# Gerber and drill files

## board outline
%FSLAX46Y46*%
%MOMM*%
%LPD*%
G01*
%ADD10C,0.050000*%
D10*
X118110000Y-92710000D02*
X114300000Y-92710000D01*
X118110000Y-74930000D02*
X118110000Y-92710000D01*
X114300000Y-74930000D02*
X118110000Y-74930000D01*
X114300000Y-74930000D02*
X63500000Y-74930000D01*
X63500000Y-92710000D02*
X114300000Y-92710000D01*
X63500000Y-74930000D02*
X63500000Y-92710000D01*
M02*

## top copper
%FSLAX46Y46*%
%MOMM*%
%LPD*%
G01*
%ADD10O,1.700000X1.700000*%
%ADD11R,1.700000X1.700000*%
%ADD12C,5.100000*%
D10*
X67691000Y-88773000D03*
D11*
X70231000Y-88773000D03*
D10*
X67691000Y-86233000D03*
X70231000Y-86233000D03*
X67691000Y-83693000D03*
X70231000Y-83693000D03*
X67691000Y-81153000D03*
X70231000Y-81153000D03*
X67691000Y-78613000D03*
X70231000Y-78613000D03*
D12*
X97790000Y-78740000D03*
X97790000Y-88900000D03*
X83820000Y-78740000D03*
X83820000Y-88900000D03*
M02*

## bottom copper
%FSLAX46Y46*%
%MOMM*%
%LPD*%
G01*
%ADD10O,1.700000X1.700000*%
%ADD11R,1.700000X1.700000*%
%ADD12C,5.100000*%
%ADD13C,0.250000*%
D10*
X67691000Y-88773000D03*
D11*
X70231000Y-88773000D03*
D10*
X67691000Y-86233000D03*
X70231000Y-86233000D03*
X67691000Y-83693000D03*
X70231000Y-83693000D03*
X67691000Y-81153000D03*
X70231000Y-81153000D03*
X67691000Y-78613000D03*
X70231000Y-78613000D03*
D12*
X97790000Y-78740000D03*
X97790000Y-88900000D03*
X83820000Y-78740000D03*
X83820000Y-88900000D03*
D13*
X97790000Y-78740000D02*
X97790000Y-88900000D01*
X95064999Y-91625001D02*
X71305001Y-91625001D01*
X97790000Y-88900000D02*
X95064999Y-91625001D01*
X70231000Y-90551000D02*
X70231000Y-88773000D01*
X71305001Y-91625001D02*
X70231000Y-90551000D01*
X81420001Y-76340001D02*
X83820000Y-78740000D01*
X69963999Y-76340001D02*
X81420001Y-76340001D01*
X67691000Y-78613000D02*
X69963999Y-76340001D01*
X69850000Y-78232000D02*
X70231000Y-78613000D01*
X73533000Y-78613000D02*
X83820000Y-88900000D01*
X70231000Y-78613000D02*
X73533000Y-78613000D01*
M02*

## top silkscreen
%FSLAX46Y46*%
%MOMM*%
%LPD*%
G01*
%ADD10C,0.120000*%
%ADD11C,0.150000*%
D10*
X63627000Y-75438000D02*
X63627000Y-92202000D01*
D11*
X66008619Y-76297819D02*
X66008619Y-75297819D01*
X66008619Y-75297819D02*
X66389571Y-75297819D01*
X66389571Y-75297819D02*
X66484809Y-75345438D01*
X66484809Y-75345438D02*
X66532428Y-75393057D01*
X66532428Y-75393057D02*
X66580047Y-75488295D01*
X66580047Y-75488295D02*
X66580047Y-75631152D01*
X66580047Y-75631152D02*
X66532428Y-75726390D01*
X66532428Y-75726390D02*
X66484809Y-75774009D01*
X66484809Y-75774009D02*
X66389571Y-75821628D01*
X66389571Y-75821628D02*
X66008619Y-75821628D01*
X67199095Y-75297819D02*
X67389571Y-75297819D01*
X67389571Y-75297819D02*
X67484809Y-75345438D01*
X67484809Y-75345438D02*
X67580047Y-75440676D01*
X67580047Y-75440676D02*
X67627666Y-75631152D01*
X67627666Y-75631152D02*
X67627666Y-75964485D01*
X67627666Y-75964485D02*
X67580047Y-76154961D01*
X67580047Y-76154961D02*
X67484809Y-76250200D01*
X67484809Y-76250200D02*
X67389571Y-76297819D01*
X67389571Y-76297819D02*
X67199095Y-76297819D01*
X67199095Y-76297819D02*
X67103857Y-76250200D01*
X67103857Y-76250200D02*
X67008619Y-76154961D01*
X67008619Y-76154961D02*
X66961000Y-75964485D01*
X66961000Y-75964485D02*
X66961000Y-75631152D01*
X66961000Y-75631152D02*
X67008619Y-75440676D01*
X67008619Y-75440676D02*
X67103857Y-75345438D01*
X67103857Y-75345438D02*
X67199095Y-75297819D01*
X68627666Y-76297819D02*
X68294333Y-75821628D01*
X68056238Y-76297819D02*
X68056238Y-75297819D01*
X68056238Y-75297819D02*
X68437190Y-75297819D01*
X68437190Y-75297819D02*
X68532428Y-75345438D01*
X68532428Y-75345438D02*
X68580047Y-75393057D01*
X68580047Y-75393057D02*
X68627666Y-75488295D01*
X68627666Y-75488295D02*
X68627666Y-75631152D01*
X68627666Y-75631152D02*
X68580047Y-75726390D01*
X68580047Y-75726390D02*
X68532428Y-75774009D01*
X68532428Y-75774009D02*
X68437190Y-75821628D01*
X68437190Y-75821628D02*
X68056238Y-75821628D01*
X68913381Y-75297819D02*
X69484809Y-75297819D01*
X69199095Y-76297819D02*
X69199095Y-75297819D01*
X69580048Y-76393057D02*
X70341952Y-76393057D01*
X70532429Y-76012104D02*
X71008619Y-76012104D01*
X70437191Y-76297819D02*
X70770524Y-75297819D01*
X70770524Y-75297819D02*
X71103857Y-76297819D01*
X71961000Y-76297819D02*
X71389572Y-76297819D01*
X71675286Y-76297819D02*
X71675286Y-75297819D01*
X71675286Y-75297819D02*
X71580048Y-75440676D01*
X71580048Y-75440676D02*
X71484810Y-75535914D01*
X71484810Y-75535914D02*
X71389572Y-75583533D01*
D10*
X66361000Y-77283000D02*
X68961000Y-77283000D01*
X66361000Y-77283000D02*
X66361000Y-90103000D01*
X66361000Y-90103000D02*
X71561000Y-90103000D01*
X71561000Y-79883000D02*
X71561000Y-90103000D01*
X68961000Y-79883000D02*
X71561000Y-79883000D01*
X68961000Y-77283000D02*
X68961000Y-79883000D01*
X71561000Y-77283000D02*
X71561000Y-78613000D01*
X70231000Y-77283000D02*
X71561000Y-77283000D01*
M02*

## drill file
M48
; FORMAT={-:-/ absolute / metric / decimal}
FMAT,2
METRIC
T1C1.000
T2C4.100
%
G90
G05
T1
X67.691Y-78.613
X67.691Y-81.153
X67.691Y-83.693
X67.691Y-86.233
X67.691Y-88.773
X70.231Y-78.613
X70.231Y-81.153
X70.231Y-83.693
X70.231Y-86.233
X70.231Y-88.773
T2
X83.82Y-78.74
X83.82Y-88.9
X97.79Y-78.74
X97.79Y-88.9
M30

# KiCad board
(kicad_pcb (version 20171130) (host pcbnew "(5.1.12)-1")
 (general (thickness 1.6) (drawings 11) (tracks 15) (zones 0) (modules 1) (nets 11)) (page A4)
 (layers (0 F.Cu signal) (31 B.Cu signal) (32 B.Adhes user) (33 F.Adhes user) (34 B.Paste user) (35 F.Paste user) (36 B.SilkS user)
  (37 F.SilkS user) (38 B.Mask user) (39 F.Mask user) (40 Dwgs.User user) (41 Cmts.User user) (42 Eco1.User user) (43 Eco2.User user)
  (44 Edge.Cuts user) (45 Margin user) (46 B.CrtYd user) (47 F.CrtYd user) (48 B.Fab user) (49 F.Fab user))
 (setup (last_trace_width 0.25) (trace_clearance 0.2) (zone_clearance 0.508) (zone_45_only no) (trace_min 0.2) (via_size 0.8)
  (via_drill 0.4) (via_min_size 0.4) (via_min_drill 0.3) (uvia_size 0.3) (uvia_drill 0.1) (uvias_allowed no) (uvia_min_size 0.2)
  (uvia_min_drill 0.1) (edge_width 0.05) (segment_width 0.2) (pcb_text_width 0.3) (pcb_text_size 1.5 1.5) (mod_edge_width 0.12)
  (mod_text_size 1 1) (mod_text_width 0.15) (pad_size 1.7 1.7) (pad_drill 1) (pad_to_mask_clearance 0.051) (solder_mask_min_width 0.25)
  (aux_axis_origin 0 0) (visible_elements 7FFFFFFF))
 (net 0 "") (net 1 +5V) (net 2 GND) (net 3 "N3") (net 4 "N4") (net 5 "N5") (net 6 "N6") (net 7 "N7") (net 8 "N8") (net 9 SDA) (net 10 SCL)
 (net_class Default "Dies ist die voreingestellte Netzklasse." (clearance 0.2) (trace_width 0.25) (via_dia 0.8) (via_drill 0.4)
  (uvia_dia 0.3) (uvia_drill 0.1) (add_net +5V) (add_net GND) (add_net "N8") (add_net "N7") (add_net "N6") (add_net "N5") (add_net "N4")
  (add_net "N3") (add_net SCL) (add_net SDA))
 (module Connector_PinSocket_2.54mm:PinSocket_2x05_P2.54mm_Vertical (layer F.Cu) (at 70.231 78.613)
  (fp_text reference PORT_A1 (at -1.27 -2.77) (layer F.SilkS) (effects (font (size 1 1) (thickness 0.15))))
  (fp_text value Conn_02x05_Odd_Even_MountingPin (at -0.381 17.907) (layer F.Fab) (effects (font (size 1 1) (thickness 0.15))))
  (fp_line (start -3.87 -1.33) (end -1.27 -1.33) (layer F.SilkS) (width 0.12))
  (fp_line (start -3.87 -1.33) (end -3.87 11.49) (layer F.SilkS) (width 0.12))
  (fp_line (start -3.87 11.49) (end 1.33 11.49) (layer F.SilkS) (width 0.12))
  (fp_line (start 1.33 1.27) (end 1.33 11.49) (layer F.SilkS) (width 0.12))
  (fp_line (start -1.27 1.27) (end 1.33 1.27) (layer F.SilkS) (width 0.12))
  (fp_line (start -1.27 -1.33) (end -1.27 1.27) (layer F.SilkS) (width 0.12))
  (fp_line (start 1.33 -1.33) (end 1.33 0) (layer F.SilkS) (width 0.12))
  (fp_line (start 0 -1.33) (end 1.33 -1.33) (layer F.SilkS) (width 0.12))
  (pad 10 thru_hole oval (at -2.54 10.16) (size 1.7 1.7) (drill 1) (layers *.Cu *.Mask) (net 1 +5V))
  (pad 9 thru_hole rect (at 0 10.16) (size 1.7 1.7) (drill 1) (layers *.Cu *.Mask) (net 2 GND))
  (pad 8 thru_hole oval (at -2.54 7.62) (size 1.7 1.7) (drill 1) (layers *.Cu *.Mask) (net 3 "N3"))
  (pad 7 thru_hole oval (at 0 7.62) (size 1.7 1.7) (drill 1) (layers *.Cu *.Mask) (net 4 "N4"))
  (pad 6 thru_hole oval (at -2.54 5.08) (size 1.7 1.7) (drill 1) (layers *.Cu *.Mask) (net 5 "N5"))
  (pad 5 thru_hole oval (at 0 5.08) (size 1.7 1.7) (drill 1) (layers *.Cu *.Mask) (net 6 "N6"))
  (pad 4 thru_hole oval (at -2.54 2.54) (size 1.7 1.7) (drill 1) (layers *.Cu *.Mask) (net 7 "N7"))
  (pad 3 thru_hole oval (at 0 2.54) (size 1.7 1.7) (drill 1) (layers *.Cu *.Mask) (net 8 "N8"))
  (pad 2 thru_hole oval (at -2.54 0) (size 1.7 1.7) (drill 1) (layers *.Cu *.Mask) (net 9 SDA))
  (pad 1 thru_hole oval (at 0 0) (size 1.7 1.7) (drill 1) (layers *.Cu *.Mask) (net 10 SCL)))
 (gr_line (start 118.11 92.71) (end 114.3 92.71) (layer Edge.Cuts) (width 0.05))
 (gr_line (start 118.11 74.93) (end 118.11 92.71) (layer Edge.Cuts) (width 0.05))
 (gr_line (start 114.3 74.93) (end 118.11 74.93) (layer Edge.Cuts) (width 0.05))
 (gr_line (start 114.3 74.93) (end 63.5 74.93) (layer Edge.Cuts) (width 0.05))
 (gr_line (start 63.5 92.71) (end 114.3 92.71) (layer Edge.Cuts) (width 0.05))
 (gr_line (start 63.5 74.93) (end 63.5 92.71) (layer Edge.Cuts) (width 0.05))
 (gr_line (start 63.627 75.438) (end 63.627 92.202) (layer F.SilkS) (width 0.12))
 (via (at 97.79 78.74) (size 5.1) (drill 4.1) (layers F.Cu B.Cu) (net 2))
 (via (at 97.79 88.9) (size 5.1) (drill 4.1) (layers F.Cu B.Cu) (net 2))
 (segment (start 97.79 78.74) (end 97.79 88.9) (width 0.25) (layer B.Cu) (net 2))
 (segment (start 95.064999 91.625001) (end 71.305001 91.625001) (width 0.25) (layer B.Cu) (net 2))
 (segment (start 97.79 88.9) (end 95.064999 91.625001) (width 0.25) (layer B.Cu) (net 2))
 (segment (start 70.231 90.551) (end 70.231 88.773) (width 0.25) (layer B.Cu) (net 2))
 (segment (start 71.305001 91.625001) (end 70.231 90.551) (width 0.25) (layer B.Cu) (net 2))
 (via (at 83.82 78.74) (size 5.1) (drill 4.1) (layers F.Cu B.Cu) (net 9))
 (segment (start 81.420001 76.340001) (end 83.82 78.74) (width 0.25) (layer B.Cu) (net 9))
 (segment (start 69.963999 76.340001) (end 81.420001 76.340001) (width 0.25) (layer B.Cu) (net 9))
 (segment (start 67.691 78.613) (end 69.963999 76.340001) (width 0.25) (layer B.Cu) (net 9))
 (via (at 83.82 88.9) (size 5.1) (drill 4.1) (layers F.Cu B.Cu) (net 10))
 (segment (start 69.85 78.232) (end 70.231 78.613) (width 0.25) (layer B.Cu) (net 10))
 (segment (start 73.533 78.613) (end 83.82 88.9) (width 0.25) (layer B.Cu) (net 10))
 (segment (start 70.231 78.613) (end 73.533 78.613) (width 0.25) (layer B.Cu) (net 10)))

